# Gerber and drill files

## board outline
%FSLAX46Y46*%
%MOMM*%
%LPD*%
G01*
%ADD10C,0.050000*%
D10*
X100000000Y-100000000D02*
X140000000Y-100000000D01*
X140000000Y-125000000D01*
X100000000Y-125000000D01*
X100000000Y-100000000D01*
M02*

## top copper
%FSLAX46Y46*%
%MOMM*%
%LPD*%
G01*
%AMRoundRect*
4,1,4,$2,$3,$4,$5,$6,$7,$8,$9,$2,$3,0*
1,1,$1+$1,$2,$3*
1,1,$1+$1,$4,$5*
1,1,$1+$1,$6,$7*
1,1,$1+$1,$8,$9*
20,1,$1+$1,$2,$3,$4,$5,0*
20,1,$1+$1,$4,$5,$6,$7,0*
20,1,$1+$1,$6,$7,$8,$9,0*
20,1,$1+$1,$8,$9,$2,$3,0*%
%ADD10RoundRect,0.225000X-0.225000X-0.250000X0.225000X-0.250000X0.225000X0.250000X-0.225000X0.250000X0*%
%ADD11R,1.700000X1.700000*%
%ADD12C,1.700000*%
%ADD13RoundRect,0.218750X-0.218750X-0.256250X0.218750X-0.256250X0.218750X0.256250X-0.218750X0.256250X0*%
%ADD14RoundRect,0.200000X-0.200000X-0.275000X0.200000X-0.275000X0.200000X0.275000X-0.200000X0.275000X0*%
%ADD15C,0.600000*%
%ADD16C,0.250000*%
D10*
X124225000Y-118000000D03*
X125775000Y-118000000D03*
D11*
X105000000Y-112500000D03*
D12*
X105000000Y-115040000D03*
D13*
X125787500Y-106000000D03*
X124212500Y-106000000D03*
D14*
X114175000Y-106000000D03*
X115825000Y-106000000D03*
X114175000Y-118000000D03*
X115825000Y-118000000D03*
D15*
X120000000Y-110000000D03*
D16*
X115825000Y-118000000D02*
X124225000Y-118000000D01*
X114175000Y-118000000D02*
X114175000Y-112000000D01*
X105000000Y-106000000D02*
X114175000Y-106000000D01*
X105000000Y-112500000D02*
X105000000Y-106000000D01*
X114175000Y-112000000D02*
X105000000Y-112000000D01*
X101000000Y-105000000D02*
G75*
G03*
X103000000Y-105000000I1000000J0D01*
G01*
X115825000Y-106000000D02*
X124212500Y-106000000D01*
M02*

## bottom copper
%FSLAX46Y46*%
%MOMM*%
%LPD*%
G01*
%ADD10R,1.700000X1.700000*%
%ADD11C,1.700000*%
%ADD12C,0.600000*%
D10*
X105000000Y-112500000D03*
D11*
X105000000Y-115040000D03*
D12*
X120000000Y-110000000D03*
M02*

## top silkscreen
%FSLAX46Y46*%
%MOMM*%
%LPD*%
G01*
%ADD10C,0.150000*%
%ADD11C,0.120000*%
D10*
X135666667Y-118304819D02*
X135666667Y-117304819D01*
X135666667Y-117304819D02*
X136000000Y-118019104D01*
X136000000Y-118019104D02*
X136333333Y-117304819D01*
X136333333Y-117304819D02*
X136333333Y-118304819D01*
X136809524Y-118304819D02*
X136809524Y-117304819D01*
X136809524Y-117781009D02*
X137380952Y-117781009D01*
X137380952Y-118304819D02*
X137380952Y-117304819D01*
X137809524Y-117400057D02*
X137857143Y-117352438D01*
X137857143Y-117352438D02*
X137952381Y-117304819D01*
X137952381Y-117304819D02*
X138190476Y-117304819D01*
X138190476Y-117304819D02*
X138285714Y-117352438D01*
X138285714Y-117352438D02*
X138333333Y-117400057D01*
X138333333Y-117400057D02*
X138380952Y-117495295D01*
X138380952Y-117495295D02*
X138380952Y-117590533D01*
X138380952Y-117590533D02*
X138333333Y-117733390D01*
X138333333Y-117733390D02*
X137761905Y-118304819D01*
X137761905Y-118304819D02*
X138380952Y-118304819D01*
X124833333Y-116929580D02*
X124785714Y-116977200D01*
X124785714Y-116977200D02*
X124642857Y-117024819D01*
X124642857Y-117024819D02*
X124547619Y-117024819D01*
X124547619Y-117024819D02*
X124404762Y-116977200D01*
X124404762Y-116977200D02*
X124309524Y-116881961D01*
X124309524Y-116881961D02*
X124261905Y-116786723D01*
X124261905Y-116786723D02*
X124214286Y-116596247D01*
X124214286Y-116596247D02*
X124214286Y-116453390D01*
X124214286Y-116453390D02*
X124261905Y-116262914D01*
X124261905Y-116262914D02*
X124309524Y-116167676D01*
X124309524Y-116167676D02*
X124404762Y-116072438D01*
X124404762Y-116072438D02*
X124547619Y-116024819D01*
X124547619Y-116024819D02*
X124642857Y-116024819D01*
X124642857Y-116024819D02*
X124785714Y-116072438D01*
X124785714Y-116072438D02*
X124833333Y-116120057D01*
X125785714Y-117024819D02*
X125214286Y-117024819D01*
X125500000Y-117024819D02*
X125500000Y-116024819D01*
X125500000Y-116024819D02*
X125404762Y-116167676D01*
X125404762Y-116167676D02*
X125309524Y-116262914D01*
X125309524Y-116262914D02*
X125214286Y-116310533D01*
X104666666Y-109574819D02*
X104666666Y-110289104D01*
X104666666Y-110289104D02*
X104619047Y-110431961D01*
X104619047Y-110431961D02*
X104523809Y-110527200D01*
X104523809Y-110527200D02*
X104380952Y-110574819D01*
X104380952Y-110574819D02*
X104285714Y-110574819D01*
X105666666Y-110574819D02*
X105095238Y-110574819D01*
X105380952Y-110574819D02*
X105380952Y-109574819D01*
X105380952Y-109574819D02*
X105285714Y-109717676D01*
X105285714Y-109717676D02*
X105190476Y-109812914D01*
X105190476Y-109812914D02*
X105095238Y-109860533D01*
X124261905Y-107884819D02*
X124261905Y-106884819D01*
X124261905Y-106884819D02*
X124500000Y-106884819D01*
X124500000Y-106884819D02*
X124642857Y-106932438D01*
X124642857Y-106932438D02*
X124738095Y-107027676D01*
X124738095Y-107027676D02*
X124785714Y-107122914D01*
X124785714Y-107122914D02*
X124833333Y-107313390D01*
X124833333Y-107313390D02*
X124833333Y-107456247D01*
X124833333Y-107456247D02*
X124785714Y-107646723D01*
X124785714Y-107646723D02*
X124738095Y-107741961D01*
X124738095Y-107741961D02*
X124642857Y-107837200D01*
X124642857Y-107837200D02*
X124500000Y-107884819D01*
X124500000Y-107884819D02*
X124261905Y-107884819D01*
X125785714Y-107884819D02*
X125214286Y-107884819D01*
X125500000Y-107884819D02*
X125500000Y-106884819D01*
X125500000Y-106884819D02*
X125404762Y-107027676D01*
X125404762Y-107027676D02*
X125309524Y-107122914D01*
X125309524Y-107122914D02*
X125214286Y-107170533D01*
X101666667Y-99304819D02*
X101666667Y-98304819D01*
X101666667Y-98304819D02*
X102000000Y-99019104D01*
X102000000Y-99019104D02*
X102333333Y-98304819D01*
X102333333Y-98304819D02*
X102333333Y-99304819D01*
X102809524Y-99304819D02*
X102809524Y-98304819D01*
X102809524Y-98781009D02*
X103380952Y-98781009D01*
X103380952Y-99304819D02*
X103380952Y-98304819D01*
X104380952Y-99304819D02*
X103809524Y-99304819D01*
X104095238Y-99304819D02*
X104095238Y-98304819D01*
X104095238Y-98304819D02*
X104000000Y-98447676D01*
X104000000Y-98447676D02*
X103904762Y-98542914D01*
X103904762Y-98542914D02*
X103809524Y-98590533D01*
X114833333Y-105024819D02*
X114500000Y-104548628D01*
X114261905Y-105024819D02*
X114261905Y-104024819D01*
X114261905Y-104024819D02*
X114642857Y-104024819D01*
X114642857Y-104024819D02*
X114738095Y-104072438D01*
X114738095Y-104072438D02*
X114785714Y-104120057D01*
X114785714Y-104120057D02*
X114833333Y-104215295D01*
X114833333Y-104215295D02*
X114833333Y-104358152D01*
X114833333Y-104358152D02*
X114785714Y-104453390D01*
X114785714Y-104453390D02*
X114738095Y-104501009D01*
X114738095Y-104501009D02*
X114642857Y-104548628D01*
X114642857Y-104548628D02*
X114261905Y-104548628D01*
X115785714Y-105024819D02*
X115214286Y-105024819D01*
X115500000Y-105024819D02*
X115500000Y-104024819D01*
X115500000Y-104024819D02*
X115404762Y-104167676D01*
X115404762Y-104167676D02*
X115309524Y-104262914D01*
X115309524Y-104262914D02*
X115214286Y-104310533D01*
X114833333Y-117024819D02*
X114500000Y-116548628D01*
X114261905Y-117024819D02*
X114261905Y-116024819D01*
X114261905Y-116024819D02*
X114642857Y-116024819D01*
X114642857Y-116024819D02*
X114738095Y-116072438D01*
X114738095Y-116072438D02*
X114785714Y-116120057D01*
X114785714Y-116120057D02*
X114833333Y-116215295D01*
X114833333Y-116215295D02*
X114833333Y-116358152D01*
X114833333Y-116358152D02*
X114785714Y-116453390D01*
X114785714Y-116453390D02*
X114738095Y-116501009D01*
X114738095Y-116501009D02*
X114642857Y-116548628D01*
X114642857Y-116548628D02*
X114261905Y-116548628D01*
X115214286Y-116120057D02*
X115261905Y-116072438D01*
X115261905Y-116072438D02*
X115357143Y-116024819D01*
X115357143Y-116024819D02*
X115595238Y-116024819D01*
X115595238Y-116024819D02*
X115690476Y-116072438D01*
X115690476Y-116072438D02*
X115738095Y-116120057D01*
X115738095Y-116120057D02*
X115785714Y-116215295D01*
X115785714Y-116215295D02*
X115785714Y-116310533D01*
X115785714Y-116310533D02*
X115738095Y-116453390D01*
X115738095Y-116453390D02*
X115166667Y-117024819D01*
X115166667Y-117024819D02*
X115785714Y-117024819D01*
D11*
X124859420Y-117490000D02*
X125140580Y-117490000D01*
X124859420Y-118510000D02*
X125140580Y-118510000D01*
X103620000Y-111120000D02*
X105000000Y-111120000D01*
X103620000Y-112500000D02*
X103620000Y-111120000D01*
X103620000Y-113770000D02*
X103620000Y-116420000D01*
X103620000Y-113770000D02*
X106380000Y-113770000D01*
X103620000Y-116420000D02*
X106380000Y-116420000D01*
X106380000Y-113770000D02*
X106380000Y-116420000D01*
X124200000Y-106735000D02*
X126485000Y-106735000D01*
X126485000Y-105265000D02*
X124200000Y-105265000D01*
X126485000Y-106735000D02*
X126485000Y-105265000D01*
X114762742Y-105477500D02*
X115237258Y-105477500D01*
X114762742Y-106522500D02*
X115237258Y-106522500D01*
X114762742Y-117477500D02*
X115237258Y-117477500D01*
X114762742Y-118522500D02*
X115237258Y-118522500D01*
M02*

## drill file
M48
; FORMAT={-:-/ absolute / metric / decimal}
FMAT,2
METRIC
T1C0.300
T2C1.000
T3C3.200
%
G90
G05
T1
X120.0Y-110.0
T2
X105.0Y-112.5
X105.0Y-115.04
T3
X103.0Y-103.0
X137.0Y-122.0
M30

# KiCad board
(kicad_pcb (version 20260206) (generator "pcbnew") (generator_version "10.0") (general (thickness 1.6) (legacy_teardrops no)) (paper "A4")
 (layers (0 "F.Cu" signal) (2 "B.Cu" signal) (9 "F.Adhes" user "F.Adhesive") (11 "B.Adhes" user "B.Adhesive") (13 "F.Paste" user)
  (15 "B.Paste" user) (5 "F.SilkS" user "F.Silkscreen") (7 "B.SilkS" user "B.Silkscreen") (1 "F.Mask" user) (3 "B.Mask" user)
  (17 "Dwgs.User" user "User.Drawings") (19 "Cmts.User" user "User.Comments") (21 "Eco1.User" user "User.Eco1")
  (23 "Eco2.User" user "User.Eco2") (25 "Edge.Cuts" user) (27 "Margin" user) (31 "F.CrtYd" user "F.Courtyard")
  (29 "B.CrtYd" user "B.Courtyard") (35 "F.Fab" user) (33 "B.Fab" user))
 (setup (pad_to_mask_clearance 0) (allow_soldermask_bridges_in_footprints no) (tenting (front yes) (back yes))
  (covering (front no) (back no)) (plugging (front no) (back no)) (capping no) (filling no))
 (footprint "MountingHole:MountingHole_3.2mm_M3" (layer "F.Cu") (at 137 122)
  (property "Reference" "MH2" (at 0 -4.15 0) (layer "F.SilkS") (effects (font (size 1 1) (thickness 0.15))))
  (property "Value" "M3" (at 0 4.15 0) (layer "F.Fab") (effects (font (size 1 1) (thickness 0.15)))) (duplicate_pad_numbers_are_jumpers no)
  (pad "" np_thru_hole circle (at 0 0) (size 3.2 3.2) (drill 3.2) (layers "*.Cu" "*.Mask")))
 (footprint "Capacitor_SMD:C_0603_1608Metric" (layer "F.Cu") (at 125 118)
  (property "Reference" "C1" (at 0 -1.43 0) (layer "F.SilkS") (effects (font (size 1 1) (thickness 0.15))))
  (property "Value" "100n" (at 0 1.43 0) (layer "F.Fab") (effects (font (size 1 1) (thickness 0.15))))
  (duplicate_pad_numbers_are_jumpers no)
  (fp_line (start -0.14058 -0.51) (end 0.14058 -0.51) (stroke (width 0.12) (type solid)) (layer "F.SilkS"))
  (fp_line (start -0.14058 0.51) (end 0.14058 0.51) (stroke (width 0.12) (type solid)) (layer "F.SilkS"))
  (pad "1" smd roundrect (at -0.775 0) (size 0.9 0.95) (layers "F.Cu" "F.Mask" "F.Paste") (roundrect_rratio 0.25) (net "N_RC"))
  (pad "2" smd roundrect (at 0.775 0) (size 0.9 0.95) (layers "F.Cu" "F.Mask" "F.Paste") (roundrect_rratio 0.25) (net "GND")))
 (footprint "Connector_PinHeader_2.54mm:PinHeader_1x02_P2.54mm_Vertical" (layer "F.Cu") (at 105 112.5)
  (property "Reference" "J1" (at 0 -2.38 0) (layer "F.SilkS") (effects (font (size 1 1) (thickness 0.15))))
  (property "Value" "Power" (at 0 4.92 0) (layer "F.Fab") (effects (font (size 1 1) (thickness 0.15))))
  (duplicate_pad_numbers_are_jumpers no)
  (fp_line (start -1.38 -1.38) (end 0 -1.38) (stroke (width 0.12) (type solid)) (layer "F.SilkS"))
  (fp_line (start -1.38 0) (end -1.38 -1.38) (stroke (width 0.12) (type solid)) (layer "F.SilkS"))
  (fp_line (start -1.38 1.27) (end -1.38 3.92) (stroke (width 0.12) (type solid)) (layer "F.SilkS"))
  (fp_line (start -1.38 1.27) (end 1.38 1.27) (stroke (width 0.12) (type solid)) (layer "F.SilkS"))
  (fp_line (start -1.38 3.92) (end 1.38 3.92) (stroke (width 0.12) (type solid)) (layer "F.SilkS"))
  (fp_line (start 1.38 1.27) (end 1.38 3.92) (stroke (width 0.12) (type solid)) (layer "F.SilkS"))
  (pad "1" thru_hole rect (at 0 0) (size 1.7 1.7) (drill 1) (layers "*.Cu" "*.Mask") (remove_unused_layers no) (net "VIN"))
  (pad "2" thru_hole circle (at 0 2.54) (size 1.7 1.7) (drill 1) (layers "*.Cu" "*.Mask") (remove_unused_layers no) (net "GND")))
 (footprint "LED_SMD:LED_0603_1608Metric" (layer "F.Cu") (at 125 106 180)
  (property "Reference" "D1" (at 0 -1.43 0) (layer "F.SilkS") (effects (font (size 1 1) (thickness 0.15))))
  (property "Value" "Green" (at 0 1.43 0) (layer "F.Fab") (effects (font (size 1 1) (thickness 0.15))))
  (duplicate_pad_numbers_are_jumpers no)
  (fp_line (start 0.8 -0.735) (end -1.485 -0.735) (stroke (width 0.12) (type solid)) (layer "F.SilkS"))
  (fp_line (start -1.485 0.735) (end 0.8 0.735) (stroke (width 0.12) (type solid)) (layer "F.SilkS"))
  (fp_line (start -1.485 -0.735) (end -1.485 0.735) (stroke (width 0.12) (type solid)) (layer "F.SilkS"))
  (pad "1" smd roundrect (at -0.7875 0) (size 0.875 0.95) (layers "F.Cu" "F.Mask" "F.Paste") (roundrect_rratio 0.25) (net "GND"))
  (pad "2" smd roundrect (at 0.7875 0) (size 0.875 0.95) (layers "F.Cu" "F.Mask" "F.Paste") (roundrect_rratio 0.25) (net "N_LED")))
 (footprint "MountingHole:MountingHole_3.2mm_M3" (layer "F.Cu") (at 103 103)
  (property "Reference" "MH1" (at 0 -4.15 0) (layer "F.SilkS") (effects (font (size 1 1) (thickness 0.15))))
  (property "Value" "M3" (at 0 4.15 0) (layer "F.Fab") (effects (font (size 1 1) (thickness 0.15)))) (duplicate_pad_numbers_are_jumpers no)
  (pad "" np_thru_hole circle (at 0 0) (size 3.2 3.2) (drill 3.2) (layers "*.Cu" "*.Mask")))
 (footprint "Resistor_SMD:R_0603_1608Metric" (layer "F.Cu") (at 115 106)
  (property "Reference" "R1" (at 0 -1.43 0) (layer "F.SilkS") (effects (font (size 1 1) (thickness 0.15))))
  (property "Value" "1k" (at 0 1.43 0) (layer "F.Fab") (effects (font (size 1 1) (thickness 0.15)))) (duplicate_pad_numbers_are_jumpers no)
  (fp_line (start -0.237258 -0.5225) (end 0.237258 -0.5225) (stroke (width 0.12) (type solid)) (layer "F.SilkS"))
  (fp_line (start -0.237258 0.5225) (end 0.237258 0.5225) (stroke (width 0.12) (type solid)) (layer "F.SilkS"))
  (pad "1" smd roundrect (at -0.825 0) (size 0.8 0.95) (layers "F.Cu" "F.Mask" "F.Paste") (roundrect_rratio 0.25) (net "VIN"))
  (pad "2" smd roundrect (at 0.825 0) (size 0.8 0.95) (layers "F.Cu" "F.Mask" "F.Paste") (roundrect_rratio 0.25) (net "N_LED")))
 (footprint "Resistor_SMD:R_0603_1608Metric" (layer "F.Cu") (at 115 118)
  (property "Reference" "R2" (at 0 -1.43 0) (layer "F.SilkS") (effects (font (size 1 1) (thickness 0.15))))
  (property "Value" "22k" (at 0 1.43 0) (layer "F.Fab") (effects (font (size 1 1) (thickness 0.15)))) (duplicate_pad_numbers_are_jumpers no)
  (fp_line (start -0.237258 -0.5225) (end 0.237258 -0.5225) (stroke (width 0.12) (type solid)) (layer "F.SilkS"))
  (fp_line (start -0.237258 0.5225) (end 0.237258 0.5225) (stroke (width 0.12) (type solid)) (layer "F.SilkS"))
  (pad "1" smd roundrect (at -0.825 0) (size 0.8 0.95) (layers "F.Cu" "F.Mask" "F.Paste") (roundrect_rratio 0.25) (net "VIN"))
  (pad "2" smd roundrect (at 0.825 0) (size 0.8 0.95) (layers "F.Cu" "F.Mask" "F.Paste") (roundrect_rratio 0.25) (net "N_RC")))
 (gr_rect (start 100 100) (end 140 125) (stroke (width 0.05) (type default)) (fill no) (layer "Edge.Cuts"))
 (segment (start 115.825 118) (end 124.225 118) (width 0.25) (layer "F.Cu") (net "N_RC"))
 (segment (start 114.175 118) (end 114.175 112) (width 0.25) (layer "F.Cu") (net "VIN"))
 (segment (start 105 106) (end 114.175 106) (width 0.25) (layer "F.Cu") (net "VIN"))
 (segment (start 105 112.5) (end 105 106) (width 0.25) (layer "F.Cu") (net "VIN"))
 (segment (start 114.175 112) (end 105 112) (width 0.25) (layer "F.Cu") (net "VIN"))
 (via (at 120 110) (size 0.6) (drill 0.3) (layers "F.Cu" "B.Cu") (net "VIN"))
 (arc (start 101 105) (mid 102 106) (end 103 105) (width 0.25) (layer "F.Cu") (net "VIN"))
 (segment (start 115.825 106) (end 124.2125 106) (width 0.25) (layer "F.Cu") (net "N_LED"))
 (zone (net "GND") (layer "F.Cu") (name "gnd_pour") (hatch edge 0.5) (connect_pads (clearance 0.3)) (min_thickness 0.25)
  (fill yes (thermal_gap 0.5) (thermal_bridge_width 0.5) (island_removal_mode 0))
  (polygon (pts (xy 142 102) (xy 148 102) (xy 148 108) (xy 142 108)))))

